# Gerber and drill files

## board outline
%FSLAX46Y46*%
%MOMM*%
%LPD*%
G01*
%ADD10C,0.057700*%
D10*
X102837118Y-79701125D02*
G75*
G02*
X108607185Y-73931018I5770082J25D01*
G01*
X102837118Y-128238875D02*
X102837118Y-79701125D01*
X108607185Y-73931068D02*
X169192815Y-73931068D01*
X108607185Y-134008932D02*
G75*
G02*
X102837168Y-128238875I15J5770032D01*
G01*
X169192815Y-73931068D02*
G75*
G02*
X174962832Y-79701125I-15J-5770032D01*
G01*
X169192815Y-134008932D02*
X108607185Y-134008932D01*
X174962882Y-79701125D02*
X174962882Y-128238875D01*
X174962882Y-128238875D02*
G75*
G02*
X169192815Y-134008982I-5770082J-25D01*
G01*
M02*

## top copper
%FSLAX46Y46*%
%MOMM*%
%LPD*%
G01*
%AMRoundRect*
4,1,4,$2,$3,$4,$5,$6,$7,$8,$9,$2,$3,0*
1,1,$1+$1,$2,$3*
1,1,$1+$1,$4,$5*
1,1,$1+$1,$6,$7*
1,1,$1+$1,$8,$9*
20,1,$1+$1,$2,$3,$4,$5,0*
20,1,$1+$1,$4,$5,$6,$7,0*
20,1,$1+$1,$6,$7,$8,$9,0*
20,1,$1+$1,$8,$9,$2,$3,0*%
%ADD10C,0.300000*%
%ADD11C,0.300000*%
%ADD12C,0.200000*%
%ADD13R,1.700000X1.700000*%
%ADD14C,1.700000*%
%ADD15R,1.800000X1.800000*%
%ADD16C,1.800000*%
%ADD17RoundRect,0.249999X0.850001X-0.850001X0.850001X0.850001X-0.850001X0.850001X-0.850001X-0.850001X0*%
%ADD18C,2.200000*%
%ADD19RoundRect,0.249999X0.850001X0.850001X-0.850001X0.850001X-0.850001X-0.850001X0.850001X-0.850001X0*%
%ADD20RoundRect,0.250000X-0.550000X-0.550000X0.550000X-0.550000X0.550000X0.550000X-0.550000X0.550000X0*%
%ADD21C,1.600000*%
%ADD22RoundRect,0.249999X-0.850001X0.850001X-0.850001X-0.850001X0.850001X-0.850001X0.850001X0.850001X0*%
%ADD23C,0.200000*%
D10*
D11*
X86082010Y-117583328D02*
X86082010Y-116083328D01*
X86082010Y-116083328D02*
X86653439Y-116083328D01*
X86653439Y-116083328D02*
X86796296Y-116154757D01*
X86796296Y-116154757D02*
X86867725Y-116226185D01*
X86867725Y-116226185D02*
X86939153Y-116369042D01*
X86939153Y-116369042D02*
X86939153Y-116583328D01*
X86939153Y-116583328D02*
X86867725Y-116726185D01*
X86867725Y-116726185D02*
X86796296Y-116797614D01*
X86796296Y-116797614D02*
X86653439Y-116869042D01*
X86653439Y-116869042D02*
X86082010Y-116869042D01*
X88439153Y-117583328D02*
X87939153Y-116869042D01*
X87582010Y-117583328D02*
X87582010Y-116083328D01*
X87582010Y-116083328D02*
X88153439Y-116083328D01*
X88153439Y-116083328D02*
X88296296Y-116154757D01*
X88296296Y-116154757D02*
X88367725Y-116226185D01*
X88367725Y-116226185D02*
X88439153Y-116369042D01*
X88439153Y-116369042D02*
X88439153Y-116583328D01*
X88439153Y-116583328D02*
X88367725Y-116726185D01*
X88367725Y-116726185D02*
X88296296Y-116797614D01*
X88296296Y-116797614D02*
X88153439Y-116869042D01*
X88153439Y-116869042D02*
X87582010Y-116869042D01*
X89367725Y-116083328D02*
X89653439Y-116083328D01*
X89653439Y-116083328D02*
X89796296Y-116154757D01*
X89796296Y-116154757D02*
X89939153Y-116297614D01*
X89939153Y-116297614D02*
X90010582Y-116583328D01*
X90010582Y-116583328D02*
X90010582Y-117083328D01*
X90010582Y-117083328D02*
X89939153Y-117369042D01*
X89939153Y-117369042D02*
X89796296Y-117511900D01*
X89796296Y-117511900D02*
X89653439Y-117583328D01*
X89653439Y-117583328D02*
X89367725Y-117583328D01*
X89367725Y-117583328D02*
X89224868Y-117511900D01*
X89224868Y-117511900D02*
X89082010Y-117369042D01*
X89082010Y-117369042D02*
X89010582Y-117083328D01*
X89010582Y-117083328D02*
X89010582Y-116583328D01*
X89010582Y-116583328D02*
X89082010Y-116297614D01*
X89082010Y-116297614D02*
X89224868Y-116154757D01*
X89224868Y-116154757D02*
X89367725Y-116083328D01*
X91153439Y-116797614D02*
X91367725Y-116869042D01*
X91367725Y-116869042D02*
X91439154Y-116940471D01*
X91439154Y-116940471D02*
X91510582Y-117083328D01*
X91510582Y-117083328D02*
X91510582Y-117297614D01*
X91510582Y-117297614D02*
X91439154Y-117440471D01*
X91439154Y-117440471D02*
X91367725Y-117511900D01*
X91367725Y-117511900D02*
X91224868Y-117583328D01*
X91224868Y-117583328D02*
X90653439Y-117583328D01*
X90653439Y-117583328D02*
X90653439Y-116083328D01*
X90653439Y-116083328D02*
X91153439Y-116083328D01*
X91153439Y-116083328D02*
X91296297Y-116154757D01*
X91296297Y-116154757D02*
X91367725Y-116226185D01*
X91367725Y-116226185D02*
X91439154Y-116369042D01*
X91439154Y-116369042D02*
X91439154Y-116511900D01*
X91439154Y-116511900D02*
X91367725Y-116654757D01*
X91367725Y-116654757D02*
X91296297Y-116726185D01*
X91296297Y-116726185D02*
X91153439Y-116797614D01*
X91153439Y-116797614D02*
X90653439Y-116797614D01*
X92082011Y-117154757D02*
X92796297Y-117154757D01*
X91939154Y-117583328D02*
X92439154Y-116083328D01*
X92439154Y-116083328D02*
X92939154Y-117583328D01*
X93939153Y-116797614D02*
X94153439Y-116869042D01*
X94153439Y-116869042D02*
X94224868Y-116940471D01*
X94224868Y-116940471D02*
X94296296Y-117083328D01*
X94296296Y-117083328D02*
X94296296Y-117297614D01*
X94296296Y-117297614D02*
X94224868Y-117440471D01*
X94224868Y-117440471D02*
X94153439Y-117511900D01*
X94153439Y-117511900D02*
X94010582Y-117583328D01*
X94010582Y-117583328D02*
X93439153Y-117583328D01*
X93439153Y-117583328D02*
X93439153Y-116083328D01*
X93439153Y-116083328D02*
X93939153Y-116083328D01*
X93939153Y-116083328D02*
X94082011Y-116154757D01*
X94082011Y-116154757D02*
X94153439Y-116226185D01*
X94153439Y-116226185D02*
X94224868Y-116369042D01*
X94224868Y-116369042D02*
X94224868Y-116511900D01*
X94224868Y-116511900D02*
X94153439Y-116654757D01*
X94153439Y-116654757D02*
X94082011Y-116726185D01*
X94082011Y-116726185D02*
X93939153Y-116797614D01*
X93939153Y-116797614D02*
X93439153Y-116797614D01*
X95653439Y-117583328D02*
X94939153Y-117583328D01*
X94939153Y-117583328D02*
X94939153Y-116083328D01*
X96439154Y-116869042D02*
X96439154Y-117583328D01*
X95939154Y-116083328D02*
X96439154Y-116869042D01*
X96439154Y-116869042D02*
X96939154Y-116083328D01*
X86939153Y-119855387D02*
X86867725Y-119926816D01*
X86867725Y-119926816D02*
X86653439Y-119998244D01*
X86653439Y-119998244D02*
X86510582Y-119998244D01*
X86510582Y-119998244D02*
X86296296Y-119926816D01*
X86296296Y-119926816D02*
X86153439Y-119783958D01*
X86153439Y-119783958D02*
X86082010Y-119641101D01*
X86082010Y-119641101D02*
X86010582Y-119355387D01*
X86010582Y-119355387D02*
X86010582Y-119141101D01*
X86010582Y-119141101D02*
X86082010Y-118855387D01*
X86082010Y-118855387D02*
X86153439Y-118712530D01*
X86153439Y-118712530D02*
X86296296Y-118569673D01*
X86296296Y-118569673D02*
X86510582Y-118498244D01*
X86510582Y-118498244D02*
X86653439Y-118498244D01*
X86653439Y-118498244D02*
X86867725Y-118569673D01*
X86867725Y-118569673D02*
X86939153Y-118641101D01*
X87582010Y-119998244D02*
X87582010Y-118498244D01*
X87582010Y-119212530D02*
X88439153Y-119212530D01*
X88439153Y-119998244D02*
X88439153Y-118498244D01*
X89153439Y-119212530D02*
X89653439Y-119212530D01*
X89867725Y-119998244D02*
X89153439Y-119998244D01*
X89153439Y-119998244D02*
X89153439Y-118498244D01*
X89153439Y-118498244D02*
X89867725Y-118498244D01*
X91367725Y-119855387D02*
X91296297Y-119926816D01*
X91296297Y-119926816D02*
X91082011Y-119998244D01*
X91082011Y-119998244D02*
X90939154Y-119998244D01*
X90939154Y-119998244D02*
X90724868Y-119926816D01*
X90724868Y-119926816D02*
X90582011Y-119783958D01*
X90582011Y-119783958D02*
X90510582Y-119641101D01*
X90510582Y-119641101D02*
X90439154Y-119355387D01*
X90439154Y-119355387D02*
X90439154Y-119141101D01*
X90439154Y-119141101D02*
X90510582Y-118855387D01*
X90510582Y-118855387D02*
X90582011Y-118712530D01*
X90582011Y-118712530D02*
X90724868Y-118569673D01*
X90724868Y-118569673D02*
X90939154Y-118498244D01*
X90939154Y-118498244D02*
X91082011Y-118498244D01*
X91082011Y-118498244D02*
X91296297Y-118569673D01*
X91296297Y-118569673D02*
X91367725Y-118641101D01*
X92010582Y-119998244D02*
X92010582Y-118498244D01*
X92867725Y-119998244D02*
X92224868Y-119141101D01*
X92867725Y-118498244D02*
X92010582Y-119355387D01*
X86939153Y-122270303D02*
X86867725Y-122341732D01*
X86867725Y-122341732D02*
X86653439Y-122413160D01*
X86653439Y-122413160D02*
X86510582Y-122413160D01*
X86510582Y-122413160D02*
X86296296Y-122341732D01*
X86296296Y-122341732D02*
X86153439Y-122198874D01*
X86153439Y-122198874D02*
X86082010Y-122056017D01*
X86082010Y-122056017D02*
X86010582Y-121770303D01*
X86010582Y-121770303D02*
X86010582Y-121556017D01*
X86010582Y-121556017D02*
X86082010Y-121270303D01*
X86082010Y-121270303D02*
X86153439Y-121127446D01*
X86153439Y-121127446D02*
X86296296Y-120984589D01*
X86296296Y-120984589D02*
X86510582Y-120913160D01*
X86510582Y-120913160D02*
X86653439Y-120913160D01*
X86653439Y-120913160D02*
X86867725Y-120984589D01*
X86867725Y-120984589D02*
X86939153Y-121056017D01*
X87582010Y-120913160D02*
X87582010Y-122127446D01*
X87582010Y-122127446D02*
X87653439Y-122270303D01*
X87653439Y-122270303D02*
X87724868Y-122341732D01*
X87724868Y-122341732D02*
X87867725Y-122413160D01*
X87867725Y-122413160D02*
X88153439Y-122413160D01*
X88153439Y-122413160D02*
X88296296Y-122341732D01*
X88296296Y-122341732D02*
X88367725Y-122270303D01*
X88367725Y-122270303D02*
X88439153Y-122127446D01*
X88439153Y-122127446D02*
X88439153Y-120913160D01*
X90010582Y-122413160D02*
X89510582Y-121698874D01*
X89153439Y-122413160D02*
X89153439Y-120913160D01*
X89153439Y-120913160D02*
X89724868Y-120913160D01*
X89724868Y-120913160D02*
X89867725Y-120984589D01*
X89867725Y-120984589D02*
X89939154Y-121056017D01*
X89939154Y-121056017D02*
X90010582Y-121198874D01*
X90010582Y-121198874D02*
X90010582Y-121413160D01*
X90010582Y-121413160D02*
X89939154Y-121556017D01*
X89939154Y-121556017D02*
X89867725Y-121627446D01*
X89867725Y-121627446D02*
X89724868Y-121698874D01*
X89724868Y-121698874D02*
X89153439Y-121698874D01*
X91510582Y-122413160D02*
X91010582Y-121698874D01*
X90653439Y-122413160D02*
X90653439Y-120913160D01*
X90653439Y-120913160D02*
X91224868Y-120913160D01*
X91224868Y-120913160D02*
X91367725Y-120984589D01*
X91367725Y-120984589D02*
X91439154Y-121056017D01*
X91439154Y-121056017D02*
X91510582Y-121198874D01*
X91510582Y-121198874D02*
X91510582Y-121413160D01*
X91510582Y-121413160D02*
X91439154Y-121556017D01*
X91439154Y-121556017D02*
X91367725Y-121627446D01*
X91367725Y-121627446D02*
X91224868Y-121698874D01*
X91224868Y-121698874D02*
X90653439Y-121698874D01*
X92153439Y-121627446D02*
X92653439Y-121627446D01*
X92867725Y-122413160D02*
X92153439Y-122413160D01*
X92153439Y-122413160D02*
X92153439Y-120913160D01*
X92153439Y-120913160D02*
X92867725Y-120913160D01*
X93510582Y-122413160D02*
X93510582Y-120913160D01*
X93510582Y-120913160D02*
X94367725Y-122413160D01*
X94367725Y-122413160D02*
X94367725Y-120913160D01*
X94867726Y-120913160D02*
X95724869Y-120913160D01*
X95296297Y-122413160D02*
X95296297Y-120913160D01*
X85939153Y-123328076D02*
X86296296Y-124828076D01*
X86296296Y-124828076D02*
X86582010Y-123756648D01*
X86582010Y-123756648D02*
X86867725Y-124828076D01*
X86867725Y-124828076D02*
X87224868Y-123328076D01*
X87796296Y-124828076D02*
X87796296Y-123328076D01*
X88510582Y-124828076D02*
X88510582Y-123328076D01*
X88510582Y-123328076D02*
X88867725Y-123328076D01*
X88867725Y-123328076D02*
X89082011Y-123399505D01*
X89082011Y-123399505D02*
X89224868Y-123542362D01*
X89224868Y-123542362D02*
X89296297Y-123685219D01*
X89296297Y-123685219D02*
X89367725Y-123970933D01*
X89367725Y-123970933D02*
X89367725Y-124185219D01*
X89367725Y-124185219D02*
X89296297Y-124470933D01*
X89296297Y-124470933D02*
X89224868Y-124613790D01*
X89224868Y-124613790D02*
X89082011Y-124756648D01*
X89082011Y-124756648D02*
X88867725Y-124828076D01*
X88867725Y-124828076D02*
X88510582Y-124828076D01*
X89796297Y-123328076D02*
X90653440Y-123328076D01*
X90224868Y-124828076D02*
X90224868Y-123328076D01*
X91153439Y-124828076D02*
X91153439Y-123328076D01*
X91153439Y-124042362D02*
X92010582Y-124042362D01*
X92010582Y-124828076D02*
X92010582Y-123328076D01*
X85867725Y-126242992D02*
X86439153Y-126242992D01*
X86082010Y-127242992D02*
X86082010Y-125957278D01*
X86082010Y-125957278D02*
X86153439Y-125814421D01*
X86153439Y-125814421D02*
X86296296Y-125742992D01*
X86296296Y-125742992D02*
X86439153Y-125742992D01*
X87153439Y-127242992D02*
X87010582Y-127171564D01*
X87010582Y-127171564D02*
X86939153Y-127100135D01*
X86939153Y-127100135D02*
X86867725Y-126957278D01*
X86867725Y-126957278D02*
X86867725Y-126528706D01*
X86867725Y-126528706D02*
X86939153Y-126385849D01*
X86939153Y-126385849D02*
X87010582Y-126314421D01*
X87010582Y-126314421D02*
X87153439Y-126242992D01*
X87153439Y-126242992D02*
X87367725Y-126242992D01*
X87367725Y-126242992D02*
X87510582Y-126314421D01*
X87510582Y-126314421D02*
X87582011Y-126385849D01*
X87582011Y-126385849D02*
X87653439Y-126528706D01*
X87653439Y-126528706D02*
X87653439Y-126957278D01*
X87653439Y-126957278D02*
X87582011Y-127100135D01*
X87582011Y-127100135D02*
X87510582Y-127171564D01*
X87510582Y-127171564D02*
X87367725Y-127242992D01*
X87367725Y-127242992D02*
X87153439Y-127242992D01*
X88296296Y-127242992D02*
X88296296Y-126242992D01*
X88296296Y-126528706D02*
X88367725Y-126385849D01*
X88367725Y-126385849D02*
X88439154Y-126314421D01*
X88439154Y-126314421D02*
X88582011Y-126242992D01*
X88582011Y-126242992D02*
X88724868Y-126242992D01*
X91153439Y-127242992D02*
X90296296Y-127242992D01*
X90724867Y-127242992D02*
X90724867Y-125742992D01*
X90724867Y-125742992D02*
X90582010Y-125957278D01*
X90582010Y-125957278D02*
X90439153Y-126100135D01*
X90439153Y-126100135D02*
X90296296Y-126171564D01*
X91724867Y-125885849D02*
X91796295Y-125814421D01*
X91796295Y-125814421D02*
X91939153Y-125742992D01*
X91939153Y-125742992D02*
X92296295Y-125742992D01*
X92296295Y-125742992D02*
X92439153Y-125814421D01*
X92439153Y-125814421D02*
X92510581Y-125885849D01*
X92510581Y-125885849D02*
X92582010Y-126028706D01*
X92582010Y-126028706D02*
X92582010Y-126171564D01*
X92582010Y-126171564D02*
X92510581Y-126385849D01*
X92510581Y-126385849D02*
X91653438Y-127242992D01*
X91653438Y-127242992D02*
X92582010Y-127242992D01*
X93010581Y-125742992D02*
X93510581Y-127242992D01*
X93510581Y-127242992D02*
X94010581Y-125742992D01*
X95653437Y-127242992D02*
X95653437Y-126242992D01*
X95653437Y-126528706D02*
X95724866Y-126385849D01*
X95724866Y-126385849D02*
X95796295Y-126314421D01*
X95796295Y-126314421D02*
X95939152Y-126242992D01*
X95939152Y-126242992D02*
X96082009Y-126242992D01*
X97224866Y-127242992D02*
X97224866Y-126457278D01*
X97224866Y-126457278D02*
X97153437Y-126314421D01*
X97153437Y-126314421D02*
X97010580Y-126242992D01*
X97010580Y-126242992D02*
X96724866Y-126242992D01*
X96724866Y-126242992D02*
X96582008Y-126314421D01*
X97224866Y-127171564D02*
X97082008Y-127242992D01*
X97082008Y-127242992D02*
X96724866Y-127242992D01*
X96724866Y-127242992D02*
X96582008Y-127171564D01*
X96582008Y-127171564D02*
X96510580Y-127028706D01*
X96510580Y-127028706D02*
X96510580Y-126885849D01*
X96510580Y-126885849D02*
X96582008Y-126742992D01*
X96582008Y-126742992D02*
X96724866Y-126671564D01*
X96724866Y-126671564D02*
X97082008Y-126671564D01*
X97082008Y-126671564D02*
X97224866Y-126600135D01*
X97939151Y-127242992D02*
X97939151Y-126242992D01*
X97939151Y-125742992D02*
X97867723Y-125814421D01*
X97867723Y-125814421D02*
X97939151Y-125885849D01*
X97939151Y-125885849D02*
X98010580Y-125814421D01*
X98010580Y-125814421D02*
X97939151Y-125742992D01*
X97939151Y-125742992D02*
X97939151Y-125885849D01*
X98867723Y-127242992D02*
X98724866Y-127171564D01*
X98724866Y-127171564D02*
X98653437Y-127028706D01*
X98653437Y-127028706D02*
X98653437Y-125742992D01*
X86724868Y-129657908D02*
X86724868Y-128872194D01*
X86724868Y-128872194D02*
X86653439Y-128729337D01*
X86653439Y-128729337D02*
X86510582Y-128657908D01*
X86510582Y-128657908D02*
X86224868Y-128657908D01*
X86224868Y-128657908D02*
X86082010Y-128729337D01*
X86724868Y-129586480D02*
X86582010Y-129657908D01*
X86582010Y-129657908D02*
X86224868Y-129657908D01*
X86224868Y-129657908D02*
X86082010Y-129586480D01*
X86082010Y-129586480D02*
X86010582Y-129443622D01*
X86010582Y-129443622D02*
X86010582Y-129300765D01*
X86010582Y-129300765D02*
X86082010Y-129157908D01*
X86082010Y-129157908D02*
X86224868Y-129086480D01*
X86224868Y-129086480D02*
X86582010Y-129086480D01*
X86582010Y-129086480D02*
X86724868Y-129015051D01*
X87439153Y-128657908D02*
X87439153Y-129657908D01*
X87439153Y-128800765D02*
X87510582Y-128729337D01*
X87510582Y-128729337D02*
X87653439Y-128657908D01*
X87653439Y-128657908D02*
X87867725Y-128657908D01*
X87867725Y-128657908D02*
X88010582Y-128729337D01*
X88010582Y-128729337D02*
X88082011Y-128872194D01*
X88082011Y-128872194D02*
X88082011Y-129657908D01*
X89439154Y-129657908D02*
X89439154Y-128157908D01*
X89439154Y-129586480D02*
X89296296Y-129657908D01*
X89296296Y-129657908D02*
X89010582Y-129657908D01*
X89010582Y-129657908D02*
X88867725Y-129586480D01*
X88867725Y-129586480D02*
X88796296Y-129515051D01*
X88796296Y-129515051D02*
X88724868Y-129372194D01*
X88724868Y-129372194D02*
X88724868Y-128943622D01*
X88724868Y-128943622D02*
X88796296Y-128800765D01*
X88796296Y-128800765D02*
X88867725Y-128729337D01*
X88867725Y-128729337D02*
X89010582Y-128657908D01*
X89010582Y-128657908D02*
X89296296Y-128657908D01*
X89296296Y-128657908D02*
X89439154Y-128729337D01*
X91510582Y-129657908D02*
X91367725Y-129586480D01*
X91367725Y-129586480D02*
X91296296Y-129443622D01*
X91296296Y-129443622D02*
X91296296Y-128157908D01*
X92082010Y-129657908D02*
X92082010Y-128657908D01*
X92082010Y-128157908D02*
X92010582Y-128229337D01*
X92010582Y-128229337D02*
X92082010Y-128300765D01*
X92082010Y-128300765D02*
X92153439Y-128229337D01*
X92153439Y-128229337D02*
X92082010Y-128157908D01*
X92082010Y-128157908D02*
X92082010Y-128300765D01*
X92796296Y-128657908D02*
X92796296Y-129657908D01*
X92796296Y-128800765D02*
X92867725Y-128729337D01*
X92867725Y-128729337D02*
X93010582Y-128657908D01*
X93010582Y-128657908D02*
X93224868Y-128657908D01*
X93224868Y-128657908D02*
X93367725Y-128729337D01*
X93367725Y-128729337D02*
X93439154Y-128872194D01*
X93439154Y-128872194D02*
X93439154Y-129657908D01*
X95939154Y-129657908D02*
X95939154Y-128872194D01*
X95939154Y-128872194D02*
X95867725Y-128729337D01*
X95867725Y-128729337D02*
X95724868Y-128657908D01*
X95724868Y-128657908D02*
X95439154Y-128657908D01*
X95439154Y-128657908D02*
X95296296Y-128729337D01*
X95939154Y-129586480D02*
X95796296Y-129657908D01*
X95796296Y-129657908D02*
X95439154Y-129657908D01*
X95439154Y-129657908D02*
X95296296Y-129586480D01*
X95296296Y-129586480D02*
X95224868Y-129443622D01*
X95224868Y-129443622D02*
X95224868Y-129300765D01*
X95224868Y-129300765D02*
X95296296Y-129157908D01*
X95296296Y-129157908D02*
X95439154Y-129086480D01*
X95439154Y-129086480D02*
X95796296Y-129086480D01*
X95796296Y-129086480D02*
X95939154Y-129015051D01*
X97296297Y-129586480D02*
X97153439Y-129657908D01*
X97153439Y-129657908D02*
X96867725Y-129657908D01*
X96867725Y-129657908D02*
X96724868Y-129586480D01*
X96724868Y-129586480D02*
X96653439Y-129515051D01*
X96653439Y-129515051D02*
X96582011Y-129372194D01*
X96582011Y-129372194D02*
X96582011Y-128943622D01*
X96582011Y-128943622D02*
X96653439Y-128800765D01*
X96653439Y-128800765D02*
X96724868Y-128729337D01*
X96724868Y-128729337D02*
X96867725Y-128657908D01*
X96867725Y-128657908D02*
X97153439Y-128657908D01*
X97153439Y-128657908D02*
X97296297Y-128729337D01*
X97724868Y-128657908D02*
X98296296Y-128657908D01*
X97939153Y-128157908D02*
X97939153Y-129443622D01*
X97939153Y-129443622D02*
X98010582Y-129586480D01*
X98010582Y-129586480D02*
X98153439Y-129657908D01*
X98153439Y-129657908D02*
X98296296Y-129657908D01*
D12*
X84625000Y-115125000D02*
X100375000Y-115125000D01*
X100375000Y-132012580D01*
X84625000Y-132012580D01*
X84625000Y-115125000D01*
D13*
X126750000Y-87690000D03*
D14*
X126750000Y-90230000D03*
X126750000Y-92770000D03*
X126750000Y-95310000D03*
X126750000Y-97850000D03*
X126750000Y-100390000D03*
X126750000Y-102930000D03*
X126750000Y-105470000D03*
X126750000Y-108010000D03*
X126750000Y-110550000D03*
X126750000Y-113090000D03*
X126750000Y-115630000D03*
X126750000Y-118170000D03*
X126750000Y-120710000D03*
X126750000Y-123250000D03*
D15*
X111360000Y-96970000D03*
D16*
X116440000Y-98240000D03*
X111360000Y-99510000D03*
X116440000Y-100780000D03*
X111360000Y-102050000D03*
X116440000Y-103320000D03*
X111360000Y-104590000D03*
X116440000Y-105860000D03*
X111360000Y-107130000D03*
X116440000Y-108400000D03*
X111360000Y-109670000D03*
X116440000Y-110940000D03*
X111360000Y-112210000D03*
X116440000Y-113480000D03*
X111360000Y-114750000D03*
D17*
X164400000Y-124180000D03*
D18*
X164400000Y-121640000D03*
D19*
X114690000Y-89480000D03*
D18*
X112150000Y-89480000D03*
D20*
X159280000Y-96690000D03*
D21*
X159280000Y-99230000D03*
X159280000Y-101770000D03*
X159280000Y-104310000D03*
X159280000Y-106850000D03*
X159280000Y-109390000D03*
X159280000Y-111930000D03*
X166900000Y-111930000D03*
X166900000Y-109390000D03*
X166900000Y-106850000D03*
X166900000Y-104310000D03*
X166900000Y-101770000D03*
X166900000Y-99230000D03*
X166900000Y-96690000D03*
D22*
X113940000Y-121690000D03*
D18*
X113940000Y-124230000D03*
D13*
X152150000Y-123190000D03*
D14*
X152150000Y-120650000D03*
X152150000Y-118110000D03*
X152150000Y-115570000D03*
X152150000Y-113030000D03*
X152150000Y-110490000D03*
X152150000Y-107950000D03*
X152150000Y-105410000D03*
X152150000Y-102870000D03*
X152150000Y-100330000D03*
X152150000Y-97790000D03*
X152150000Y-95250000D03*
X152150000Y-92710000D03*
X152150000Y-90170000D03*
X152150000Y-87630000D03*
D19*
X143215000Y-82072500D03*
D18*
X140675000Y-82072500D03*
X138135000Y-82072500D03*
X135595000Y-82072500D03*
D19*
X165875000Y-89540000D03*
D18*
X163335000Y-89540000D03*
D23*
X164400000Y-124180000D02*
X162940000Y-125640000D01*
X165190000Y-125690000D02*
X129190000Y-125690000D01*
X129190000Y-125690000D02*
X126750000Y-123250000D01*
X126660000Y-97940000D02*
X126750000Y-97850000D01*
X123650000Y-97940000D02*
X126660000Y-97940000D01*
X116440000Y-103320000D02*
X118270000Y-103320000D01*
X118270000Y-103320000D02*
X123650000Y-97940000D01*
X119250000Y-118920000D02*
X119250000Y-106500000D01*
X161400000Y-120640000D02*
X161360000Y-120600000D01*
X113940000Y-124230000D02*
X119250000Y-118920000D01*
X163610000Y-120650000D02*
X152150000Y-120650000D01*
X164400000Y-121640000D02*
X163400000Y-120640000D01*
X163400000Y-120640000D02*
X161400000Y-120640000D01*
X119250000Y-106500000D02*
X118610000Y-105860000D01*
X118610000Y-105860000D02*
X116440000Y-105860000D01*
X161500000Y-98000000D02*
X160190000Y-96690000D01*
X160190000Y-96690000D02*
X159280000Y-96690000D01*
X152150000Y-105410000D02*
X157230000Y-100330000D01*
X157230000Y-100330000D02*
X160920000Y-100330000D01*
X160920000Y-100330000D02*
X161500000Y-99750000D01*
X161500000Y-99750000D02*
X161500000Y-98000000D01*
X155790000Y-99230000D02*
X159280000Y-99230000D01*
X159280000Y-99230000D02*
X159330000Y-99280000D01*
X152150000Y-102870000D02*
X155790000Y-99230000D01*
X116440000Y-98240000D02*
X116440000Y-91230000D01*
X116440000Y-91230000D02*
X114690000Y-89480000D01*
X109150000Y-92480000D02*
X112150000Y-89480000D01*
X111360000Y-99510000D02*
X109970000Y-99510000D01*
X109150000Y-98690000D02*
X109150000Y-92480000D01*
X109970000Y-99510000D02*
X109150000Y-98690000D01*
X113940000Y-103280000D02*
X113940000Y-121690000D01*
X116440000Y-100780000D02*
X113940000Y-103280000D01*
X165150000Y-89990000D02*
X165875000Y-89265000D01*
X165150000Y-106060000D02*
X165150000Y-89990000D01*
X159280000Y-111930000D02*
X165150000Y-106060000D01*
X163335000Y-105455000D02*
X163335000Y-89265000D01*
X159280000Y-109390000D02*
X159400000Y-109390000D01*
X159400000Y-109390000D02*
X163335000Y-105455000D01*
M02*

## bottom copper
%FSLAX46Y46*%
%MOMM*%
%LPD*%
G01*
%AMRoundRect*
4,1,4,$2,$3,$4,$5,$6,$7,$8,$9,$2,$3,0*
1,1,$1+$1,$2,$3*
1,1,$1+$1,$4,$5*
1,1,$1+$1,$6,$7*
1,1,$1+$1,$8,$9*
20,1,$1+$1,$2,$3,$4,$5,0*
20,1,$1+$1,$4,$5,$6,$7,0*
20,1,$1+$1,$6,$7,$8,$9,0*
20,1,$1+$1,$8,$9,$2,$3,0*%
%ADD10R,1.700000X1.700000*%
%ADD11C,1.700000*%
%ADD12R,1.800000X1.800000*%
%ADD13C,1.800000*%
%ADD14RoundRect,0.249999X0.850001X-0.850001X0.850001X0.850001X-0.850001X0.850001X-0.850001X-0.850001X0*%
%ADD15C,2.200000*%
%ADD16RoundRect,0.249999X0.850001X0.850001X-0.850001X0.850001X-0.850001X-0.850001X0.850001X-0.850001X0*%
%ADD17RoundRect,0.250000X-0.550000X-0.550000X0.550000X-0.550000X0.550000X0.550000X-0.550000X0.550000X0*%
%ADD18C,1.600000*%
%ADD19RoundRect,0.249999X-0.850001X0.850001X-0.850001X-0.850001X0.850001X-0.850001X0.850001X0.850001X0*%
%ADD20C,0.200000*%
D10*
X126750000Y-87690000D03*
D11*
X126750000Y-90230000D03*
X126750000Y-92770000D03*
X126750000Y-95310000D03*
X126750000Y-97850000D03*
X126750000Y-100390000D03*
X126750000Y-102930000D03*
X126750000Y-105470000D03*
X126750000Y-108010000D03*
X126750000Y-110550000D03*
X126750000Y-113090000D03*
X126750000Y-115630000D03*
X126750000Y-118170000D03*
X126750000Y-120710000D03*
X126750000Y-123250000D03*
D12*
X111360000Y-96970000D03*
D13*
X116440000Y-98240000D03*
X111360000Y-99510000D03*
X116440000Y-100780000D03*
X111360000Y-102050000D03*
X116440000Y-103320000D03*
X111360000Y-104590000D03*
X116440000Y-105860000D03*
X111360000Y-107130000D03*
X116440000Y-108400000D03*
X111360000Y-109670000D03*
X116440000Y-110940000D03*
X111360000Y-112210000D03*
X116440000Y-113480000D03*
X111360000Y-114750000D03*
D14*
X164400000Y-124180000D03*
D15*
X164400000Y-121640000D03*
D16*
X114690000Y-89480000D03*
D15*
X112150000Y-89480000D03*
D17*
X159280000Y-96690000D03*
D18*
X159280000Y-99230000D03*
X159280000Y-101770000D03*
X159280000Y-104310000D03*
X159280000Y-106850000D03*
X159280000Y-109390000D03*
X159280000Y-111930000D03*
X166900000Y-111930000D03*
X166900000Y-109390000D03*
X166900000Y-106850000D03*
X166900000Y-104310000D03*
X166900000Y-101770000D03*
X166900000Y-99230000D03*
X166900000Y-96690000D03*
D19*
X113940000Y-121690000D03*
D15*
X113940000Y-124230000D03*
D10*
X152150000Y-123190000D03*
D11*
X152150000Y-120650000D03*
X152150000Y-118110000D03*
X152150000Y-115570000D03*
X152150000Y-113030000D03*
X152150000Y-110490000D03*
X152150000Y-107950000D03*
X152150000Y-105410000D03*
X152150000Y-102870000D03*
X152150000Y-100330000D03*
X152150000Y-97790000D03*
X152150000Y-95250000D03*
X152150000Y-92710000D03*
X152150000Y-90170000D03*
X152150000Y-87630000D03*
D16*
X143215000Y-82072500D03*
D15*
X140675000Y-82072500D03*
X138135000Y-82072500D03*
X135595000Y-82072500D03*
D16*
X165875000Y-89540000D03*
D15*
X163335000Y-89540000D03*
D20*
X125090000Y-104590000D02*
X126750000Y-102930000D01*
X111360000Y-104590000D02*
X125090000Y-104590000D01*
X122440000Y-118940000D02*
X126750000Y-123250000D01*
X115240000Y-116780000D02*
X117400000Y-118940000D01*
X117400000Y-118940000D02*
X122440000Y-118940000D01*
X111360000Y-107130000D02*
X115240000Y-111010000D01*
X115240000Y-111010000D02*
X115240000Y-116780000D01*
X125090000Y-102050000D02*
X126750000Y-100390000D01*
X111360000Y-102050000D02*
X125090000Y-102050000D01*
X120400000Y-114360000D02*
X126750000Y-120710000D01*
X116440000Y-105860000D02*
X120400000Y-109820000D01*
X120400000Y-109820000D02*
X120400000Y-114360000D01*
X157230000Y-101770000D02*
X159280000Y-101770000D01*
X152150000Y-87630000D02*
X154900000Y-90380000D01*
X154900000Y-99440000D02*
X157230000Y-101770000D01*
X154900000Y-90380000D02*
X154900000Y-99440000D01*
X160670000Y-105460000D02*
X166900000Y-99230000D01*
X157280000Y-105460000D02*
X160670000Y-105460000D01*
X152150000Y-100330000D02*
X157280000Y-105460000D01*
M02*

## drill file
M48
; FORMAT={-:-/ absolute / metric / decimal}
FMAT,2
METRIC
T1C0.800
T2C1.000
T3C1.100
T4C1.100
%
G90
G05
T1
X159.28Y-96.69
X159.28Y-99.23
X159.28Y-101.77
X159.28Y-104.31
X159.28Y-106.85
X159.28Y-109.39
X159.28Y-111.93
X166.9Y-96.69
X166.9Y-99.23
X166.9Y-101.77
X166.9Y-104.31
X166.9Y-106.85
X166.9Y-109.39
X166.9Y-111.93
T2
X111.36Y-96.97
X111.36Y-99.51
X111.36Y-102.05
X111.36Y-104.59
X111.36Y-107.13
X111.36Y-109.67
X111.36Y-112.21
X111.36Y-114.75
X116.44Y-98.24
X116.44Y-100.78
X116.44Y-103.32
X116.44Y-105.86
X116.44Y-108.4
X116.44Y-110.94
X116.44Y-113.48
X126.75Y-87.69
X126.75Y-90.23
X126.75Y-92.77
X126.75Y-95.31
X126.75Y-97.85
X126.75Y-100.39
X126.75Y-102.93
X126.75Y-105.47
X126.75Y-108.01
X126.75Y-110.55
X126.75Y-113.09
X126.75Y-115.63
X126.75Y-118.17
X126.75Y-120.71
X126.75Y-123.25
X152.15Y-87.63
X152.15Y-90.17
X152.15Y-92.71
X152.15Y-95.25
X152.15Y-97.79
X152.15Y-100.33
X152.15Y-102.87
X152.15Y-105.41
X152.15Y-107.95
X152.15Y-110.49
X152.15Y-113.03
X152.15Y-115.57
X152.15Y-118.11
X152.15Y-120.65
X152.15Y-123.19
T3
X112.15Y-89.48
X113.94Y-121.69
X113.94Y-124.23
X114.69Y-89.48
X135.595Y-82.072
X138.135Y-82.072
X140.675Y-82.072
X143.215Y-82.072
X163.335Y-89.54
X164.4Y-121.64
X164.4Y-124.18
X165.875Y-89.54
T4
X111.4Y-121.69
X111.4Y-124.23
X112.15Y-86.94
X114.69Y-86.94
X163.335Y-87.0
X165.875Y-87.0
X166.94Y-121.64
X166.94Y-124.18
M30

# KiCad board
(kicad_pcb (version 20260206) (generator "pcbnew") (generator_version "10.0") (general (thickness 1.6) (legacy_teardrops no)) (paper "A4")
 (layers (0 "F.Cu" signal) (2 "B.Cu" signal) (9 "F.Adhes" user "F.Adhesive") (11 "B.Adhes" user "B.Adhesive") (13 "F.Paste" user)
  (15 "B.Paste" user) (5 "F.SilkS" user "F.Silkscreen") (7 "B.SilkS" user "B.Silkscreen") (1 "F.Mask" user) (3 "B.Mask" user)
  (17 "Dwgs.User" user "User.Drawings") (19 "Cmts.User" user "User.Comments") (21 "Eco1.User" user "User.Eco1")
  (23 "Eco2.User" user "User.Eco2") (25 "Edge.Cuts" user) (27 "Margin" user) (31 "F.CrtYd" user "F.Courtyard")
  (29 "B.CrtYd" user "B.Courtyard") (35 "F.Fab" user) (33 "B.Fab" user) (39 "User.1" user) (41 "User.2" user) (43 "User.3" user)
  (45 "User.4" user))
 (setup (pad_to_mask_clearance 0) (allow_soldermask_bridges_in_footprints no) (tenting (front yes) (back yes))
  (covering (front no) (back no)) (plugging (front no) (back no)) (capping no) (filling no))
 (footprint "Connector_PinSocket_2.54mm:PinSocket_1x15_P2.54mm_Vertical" (layer "F.Cu") (at 126.75 87.69)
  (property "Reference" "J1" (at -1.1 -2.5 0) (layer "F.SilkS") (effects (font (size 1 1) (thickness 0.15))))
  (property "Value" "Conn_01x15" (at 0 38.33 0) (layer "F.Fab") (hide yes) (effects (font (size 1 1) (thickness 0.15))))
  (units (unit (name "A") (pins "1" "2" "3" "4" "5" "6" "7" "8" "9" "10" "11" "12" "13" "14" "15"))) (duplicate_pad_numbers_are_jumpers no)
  (pad "1" thru_hole rect (at 0 0) (size 1.7 1.7) (drill 1) (layers "*.Cu" "*.Mask") (remove_unused_layers no) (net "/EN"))
  (pad "2" thru_hole circle (at 0 2.54) (size 1.7 1.7) (drill 1) (layers "*.Cu" "*.Mask") (remove_unused_layers no) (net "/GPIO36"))
  (pad "3" thru_hole circle (at 0 5.08) (size 1.7 1.7) (drill 1) (layers "*.Cu" "*.Mask") (remove_unused_layers no) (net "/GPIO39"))
  (pad "4" thru_hole circle (at 0 7.62) (size 1.7 1.7) (drill 1) (layers "*.Cu" "*.Mask") (remove_unused_layers no) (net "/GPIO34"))
  (pad "5" thru_hole circle (at 0 10.16) (size 1.7 1.7) (drill 1) (layers "*.Cu" "*.Mask") (remove_unused_layers no) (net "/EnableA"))
  (pad "6" thru_hole circle (at 0 12.7) (size 1.7 1.7) (drill 1) (layers "*.Cu" "*.Mask") (remove_unused_layers no) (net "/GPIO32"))
  (pad "7" thru_hole circle (at 0 15.24) (size 1.7 1.7) (drill 1) (layers "*.Cu" "*.Mask") (remove_unused_layers no) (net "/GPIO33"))
  (pad "8" thru_hole circle (at 0 17.78) (size 1.7 1.7) (drill 1) (layers "*.Cu" "*.Mask") (remove_unused_layers no) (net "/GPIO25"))
  (pad "9" thru_hole circle (at 0 20.32) (size 1.7 1.7) (drill 1) (layers "*.Cu" "*.Mask") (remove_unused_layers no) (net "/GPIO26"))
  (pad "10" thru_hole circle (at 0 22.86) (size 1.7 1.7) (drill 1) (layers "*.Cu" "*.Mask") (remove_unused_layers no) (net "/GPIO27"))
  (pad "11" thru_hole circle (at 0 25.4) (size 1.7 1.7) (drill 1) (layers "*.Cu" "*.Mask") (remove_unused_layers no) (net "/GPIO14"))
  (pad "12" thru_hole circle (at 0 27.94) (size 1.7 1.7) (drill 1) (layers "*.Cu" "*.Mask") (remove_unused_layers no) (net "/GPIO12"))
  (pad "13" thru_hole circle (at 0 30.48) (size 1.7 1.7) (drill 1) (layers "*.Cu" "*.Mask") (remove_unused_layers no) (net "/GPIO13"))
  (pad "14" thru_hole circle (at 0 33.02) (size 1.7 1.7) (drill 1) (layers "*.Cu" "*.Mask") (remove_unused_layers no) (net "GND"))
  (pad "15" thru_hole circle (at 0 35.56) (size 1.7 1.7) (drill 1) (layers "*.Cu" "*.Mask") (remove_unused_layers no) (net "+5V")))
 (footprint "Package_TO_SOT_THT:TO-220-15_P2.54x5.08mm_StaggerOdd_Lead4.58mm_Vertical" (layer "F.Cu") (at 111.36 96.97 -90)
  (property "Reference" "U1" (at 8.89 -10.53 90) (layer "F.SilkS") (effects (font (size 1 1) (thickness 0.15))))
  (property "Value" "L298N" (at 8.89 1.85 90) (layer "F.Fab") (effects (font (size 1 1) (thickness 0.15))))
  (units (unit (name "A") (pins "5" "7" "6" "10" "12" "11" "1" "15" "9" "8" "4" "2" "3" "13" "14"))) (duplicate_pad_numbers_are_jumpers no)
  (pad "1" thru_hole rect (at 0 0 270) (size 1.8 1.8) (drill 1) (layers "*.Cu" "*.Mask") (remove_unused_layers no)
   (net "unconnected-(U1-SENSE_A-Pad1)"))
  (pad "2" thru_hole circle (at 1.27 -5.08 270) (size 1.8 1.8) (drill 1) (layers "*.Cu" "*.Mask") (remove_unused_layers no)
   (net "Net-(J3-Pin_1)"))
  (pad "3" thru_hole circle (at 2.54 0 270) (size 1.8 1.8) (drill 1) (layers "*.Cu" "*.Mask") (remove_unused_layers no)
   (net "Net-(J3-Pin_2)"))
  (pad "4" thru_hole circle (at 3.81 -5.08 270) (size 1.8 1.8) (drill 1) (layers "*.Cu" "*.Mask") (remove_unused_layers no) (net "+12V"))
  (pad "5" thru_hole circle (at 5.08 0 270) (size 1.8 1.8) (drill 1) (layers "*.Cu" "*.Mask") (remove_unused_layers no) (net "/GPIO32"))
  (pad "6" thru_hole circle (at 6.35 -5.08 270) (size 1.8 1.8) (drill 1) (layers "*.Cu" "*.Mask") (remove_unused_layers no) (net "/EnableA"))
  (pad "7" thru_hole circle (at 7.62 0 270) (size 1.8 1.8) (drill 1) (layers "*.Cu" "*.Mask") (remove_unused_layers no) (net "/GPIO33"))
  (pad "8" thru_hole circle (at 8.89 -5.08 270) (size 1.8 1.8) (drill 1) (layers "*.Cu" "*.Mask") (remove_unused_layers no) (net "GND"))
  (pad "9" thru_hole circle (at 10.16 0 270) (size 1.8 1.8) (drill 1) (layers "*.Cu" "*.Mask") (remove_unused_layers no) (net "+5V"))
  (pad "10" thru_hole circle (at 11.43 -5.08 270) (size 1.8 1.8) (drill 1) (layers "*.Cu" "*.Mask") (remove_unused_layers no)
   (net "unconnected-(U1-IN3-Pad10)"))
  (pad "11" thru_hole circle (at 12.7 0 270) (size 1.8 1.8) (drill 1) (layers "*.Cu" "*.Mask") (remove_unused_layers no)
   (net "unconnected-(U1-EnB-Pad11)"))
  (pad "12" thru_hole circle (at 13.97 -5.08 270) (size 1.8 1.8) (drill 1) (layers "*.Cu" "*.Mask") (remove_unused_layers no)
   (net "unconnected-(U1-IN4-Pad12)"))
  (pad "13" thru_hole circle (at 15.24 0 270) (size 1.8 1.8) (drill 1) (layers "*.Cu" "*.Mask") (remove_unused_layers no)
   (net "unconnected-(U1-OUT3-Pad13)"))
  (pad "14" thru_hole circle (at 16.51 -5.08 270) (size 1.8 1.8) (drill 1) (layers "*.Cu" "*.Mask") (remove_unused_layers no)
   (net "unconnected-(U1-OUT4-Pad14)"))
  (pad "15" thru_hole circle (at 17.78 0 270) (size 1.8 1.8) (drill 1) (layers "*.Cu" "*.Mask") (remove_unused_layers no)
   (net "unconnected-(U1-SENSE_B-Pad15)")))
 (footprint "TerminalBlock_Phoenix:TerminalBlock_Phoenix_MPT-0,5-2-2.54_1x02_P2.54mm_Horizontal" (layer "F.Cu") (at 164.4 124.18 90)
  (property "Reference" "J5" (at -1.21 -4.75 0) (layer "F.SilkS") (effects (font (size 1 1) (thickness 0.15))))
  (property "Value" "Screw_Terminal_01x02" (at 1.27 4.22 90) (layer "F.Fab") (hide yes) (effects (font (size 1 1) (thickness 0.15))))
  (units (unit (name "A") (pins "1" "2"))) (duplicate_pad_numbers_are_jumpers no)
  (pad "" np_thru_hole circle (at 0 2.54 90) (size 1.1 1.1) (drill 1.1) (layers "*.Cu" "*.Mask"))
  (pad "" np_thru_hole circle (at 2.54 2.54 90) (size 1.1 1.1) (drill 1.1) (layers "*.Cu" "*.Mask"))
  (pad "1" thru_hole roundrect (at 0 0 90) (size 2.2 2.2) (drill 1.1) (layers "*.Cu" "*.Mask") (remove_unused_layers no)
   (roundrect_rratio 0.113636) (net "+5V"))
  (pad "2" thru_hole circle (at 2.54 0 90) (size 2.2 2.2) (drill 1.1) (layers "*.Cu" "*.Mask") (remove_unused_layers no) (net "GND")))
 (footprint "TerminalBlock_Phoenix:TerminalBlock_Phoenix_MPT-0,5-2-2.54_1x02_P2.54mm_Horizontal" (layer "F.Cu") (at 114.69 89.48 180)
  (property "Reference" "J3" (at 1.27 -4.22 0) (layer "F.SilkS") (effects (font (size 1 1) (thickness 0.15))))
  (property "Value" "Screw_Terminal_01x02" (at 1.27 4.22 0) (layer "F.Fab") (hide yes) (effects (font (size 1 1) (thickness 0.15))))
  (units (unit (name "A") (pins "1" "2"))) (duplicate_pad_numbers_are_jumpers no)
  (pad "" np_thru_hole circle (at 0 2.54 180) (size 1.1 1.1) (drill 1.1) (layers "*.Cu" "*.Mask"))
  (pad "" np_thru_hole circle (at 2.54 2.54 180) (size 1.1 1.1) (drill 1.1) (layers "*.Cu" "*.Mask"))
  (pad "1" thru_hole roundrect (at 0 0 180) (size 2.2 2.2) (drill 1.1) (layers "*.Cu" "*.Mask") (remove_unused_layers no)
   (roundrect_rratio 0.113636) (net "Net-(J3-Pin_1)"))
  (pad "2" thru_hole circle (at 2.54 0 180) (size 2.2 2.2) (drill 1.1) (layers "*.Cu" "*.Mask") (remove_unused_layers no)
   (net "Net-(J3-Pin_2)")))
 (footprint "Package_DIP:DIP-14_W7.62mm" (layer "F.Cu") (at 159.28 96.69)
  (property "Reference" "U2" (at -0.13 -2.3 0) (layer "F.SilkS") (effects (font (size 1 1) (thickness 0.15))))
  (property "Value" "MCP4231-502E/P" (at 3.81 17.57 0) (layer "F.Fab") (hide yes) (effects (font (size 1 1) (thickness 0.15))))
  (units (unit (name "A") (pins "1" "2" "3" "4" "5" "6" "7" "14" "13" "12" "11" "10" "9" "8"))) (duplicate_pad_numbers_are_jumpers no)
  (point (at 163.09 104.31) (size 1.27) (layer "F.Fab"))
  (pad "1" thru_hole roundrect (at 0 0) (size 1.6 1.6) (drill 0.8) (layers "*.Cu" "*.Mask") (remove_unused_layers no)
   (roundrect_rratio 0.15625) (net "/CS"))
  (pad "2" thru_hole circle (at 0 2.54) (size 1.6 1.6) (drill 0.8) (layers "*.Cu" "*.Mask") (remove_unused_layers no) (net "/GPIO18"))
  (pad "3" thru_hole circle (at 0 5.08) (size 1.6 1.6) (drill 0.8) (layers "*.Cu" "*.Mask") (remove_unused_layers no) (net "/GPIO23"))
  (pad "4" thru_hole circle (at 0 7.62) (size 1.6 1.6) (drill 0.8) (layers "*.Cu" "*.Mask") (remove_unused_layers no) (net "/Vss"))
  (pad "5" thru_hole circle (at 0 10.16) (size 1.6 1.6) (drill 0.8) (layers "*.Cu" "*.Mask") (remove_unused_layers no)
   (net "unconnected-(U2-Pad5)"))
  (pad "6" thru_hole circle (at 0 12.7) (size 1.6 1.6) (drill 0.8) (layers "*.Cu" "*.Mask") (remove_unused_layers no) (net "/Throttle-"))
  (pad "7" thru_hole circle (at 0 15.24) (size 1.6 1.6) (drill 0.8) (layers "*.Cu" "*.Mask") (remove_unused_layers no) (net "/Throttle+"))
  (pad "8" thru_hole circle (at 7.62 15.24) (size 1.6 1.6) (drill 0.8) (layers "*.Cu" "*.Mask") (remove_unused_layers no)
   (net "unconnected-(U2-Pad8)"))
  (pad "9" thru_hole circle (at 7.62 12.7) (size 1.6 1.6) (drill 0.8) (layers "*.Cu" "*.Mask") (remove_unused_layers no)
   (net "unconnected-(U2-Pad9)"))
  (pad "10" thru_hole circle (at 7.62 10.16) (size 1.6 1.6) (drill 0.8) (layers "*.Cu" "*.Mask") (remove_unused_layers no)
   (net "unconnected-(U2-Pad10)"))
  (pad "11" thru_hole circle (at 7.62 7.62) (size 1.6 1.6) (drill 0.8) (layers "*.Cu" "*.Mask") (remove_unused_layers no) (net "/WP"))
  (pad "12" thru_hole circle (at 7.62 5.08) (size 1.6 1.6) (drill 0.8) (layers "*.Cu" "*.Mask") (remove_unused_layers no) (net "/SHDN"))
  (pad "13" thru_hole circle (at 7.62 2.54) (size 1.6 1.6) (drill 0.8) (layers "*.Cu" "*.Mask") (remove_unused_layers no) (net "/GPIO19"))
  (pad "14" thru_hole circle (at 7.62 0) (size 1.6 1.6) (drill 0.8) (layers "*.Cu" "*.Mask") (remove_unused_layers no) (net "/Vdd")))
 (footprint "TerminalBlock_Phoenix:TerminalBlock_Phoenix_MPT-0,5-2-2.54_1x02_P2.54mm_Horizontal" (layer "F.Cu") (at 113.94 121.69 -90)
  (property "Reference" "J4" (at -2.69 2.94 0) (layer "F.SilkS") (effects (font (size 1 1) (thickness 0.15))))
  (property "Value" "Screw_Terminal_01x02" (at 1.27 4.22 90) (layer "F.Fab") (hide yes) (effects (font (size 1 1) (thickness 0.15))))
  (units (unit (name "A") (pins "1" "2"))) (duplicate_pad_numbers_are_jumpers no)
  (pad "" np_thru_hole circle (at 0 2.54 270) (size 1.1 1.1) (drill 1.1) (layers "*.Cu" "*.Mask"))
  (pad "" np_thru_hole circle (at 2.54 2.54 270) (size 1.1 1.1) (drill 1.1) (layers "*.Cu" "*.Mask"))
  (pad "1" thru_hole roundrect (at 0 0 270) (size 2.2 2.2) (drill 1.1) (layers "*.Cu" "*.Mask") (remove_unused_layers no)
   (roundrect_rratio 0.113636) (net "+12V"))
  (pad "2" thru_hole circle (at 2.54 0 270) (size 2.2 2.2) (drill 1.1) (layers "*.Cu" "*.Mask") (remove_unused_layers no) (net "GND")))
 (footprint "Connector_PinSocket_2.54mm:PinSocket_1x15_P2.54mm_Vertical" (layer "F.Cu") (at 152.15 123.19 180)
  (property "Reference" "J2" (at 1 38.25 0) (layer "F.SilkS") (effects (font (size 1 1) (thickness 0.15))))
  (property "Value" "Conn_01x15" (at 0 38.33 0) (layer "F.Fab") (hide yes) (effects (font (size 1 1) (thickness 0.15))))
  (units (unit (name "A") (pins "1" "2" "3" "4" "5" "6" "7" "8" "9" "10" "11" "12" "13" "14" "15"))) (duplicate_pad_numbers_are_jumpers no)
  (pad "1" thru_hole rect (at 0 0 180) (size 1.7 1.7) (drill 1) (layers "*.Cu" "*.Mask") (remove_unused_layers no) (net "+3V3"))
  (pad "2" thru_hole circle (at 0 2.54 180) (size 1.7 1.7) (drill 1) (layers "*.Cu" "*.Mask") (remove_unused_layers no) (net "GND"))
  (pad "3" thru_hole circle (at 0 5.08 180) (size 1.7 1.7) (drill 1) (layers "*.Cu" "*.Mask") (remove_unused_layers no) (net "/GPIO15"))
  (pad "4" thru_hole circle (at 0 7.62 180) (size 1.7 1.7) (drill 1) (layers "*.Cu" "*.Mask") (remove_unused_layers no) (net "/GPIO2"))
  (pad "5" thru_hole circle (at 0 10.16 180) (size 1.7 1.7) (drill 1) (layers "*.Cu" "*.Mask") (remove_unused_layers no) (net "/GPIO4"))
  (pad "6" thru_hole circle (at 0 12.7 180) (size 1.7 1.7) (drill 1) (layers "*.Cu" "*.Mask") (remove_unused_layers no) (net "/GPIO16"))
  (pad "7" thru_hole circle (at 0 15.24 180) (size 1.7 1.7) (drill 1) (layers "*.Cu" "*.Mask") (remove_unused_layers no) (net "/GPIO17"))
  (pad "8" thru_hole circle (at 0 17.78 180) (size 1.7 1.7) (drill 1) (layers "*.Cu" "*.Mask") (remove_unused_layers no) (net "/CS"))
  (pad "9" thru_hole circle (at 0 20.32 180) (size 1.7 1.7) (drill 1) (layers "*.Cu" "*.Mask") (remove_unused_layers no) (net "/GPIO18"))
  (pad "10" thru_hole circle (at 0 22.86 180) (size 1.7 1.7) (drill 1) (layers "*.Cu" "*.Mask") (remove_unused_layers no) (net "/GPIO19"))
  (pad "11" thru_hole circle (at 0 25.4 180) (size 1.7 1.7) (drill 1) (layers "*.Cu" "*.Mask") (remove_unused_layers no) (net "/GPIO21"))
  (pad "12" thru_hole circle (at 0 27.94 180) (size 1.7 1.7) (drill 1) (layers "*.Cu" "*.Mask") (remove_unused_layers no) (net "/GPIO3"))
  (pad "13" thru_hole circle (at 0 30.48 180) (size 1.7 1.7) (drill 1) (layers "*.Cu" "*.Mask") (remove_unused_layers no) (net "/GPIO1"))
  (pad "14" thru_hole circle (at 0 33.02 180) (size 1.7 1.7) (drill 1) (layers "*.Cu" "*.Mask") (remove_unused_layers no) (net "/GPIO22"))
  (pad "15" thru_hole circle (at 0 35.56 180) (size 1.7 1.7) (drill 1) (layers "*.Cu" "*.Mask") (remove_unused_layers no) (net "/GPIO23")))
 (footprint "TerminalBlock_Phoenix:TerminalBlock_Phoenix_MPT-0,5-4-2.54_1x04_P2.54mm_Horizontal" (layer "F.Cu") (at 143.215 82.0725 180)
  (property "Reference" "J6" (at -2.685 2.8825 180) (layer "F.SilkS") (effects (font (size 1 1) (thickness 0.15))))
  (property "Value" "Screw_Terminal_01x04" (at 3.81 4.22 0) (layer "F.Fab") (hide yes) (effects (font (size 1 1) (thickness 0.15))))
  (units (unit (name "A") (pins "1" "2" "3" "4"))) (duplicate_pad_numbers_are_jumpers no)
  (pad "1" thru_hole roundrect (at 0 0 180) (size 2.2 2.2) (drill 1.1) (layers "*.Cu" "*.Mask") (remove_unused_layers no)
   (roundrect_rratio 0.113636) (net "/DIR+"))
  (pad "2" thru_hole circle (at 2.54 0 180) (size 2.2 2.2) (drill 1.1) (layers "*.Cu" "*.Mask") (remove_unused_layers no) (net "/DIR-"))
  (pad "3" thru_hole circle (at 5.08 0 180) (size 2.2 2.2) (drill 1.1) (layers "*.Cu" "*.Mask") (remove_unused_layers no) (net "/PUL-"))
  (pad "4" thru_hole circle (at 7.62 0 180) (size 2.2 2.2) (drill 1.1) (layers "*.Cu" "*.Mask") (remove_unused_layers no) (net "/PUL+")))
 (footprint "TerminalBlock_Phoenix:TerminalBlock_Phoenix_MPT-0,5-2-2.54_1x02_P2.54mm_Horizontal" (layer "F.Cu") (at 165.875 89.54 180)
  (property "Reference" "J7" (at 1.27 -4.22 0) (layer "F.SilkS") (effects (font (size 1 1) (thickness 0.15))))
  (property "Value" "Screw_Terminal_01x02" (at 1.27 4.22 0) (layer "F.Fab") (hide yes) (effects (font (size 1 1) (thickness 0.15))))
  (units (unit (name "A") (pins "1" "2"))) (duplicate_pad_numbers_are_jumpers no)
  (pad "" np_thru_hole circle (at 0 2.54 180) (size 1.1 1.1) (drill 1.1) (layers "*.Cu" "*.Mask"))
  (pad "" np_thru_hole circle (at 2.54 2.54 180) (size 1.1 1.1) (drill 1.1) (layers "*.Cu" "*.Mask"))
  (pad "1" thru_hole roundrect (at 0 0 180) (size 2.2 2.2) (drill 1.1) (layers "*.Cu" "*.Mask") (remove_unused_layers no)
   (roundrect_rratio 0.113636) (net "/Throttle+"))
  (pad "2" thru_hole circle (at 2.54 0 180) (size 2.2 2.2) (drill 1.1) (layers "*.Cu" "*.Mask") (remove_unused_layers no) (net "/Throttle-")))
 (gr_arc (start 102.837118 79.701125) (mid 104.527131 75.621071) (end 108.607185 73.931068) (stroke (width 0.0577) (type default))
  (layer "Edge.Cuts"))
 (gr_line (start 102.837118 128.238875) (end 102.837118 79.701125) (stroke (width 0.0577) (type default)) (layer "Edge.Cuts"))
 (gr_line (start 108.607185 73.931068) (end 169.192815 73.931068) (stroke (width 0.0577) (type default)) (layer "Edge.Cuts"))
 (gr_arc (start 108.607185 134.008932) (mid 104.527139 132.318921) (end 102.837118 128.238875) (stroke (width 0.0577) (type default))
  (layer "Edge.Cuts"))
 (gr_arc (start 169.192815 73.931068) (mid 173.272861 75.621079) (end 174.962882 79.701125) (stroke (width 0.0577) (type default))
  (layer "Edge.Cuts"))
 (gr_line (start 169.192815 134.008932) (end 108.607185 134.008932) (stroke (width 0.0577) (type default)) (layer "Edge.Cuts"))
 (gr_line (start 174.962882 79.701125) (end 174.962882 128.238875) (stroke (width 0.0577) (type default)) (layer "Edge.Cuts"))
 (gr_arc (start 174.962882 128.238875) (mid 173.272869 132.318929) (end 169.192815 134.008932) (stroke (width 0.0577) (type default))
  (layer "Edge.Cuts"))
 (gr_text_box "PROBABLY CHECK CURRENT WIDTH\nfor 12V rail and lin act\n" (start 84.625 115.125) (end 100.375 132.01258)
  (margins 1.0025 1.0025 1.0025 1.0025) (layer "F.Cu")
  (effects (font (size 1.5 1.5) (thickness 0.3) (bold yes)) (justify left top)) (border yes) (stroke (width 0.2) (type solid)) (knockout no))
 (segment (start 125.09 104.59) (end 126.75 102.93) (width 0.2) (layer "B.Cu") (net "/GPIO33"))
 (segment (start 111.36 104.59) (end 125.09 104.59) (width 0.2) (layer "B.Cu") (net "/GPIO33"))
 (segment (start 164.4 124.18) (end 162.94 125.64) (width 0.2) (layer "F.Cu") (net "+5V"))
 (segment (start 165.19 125.69) (end 129.19 125.69) (width 0.2) (layer "F.Cu") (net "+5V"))
 (segment (start 129.19 125.69) (end 126.75 123.25) (width 0.2) (layer "F.Cu") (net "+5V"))
 (segment (start 122.44 118.94) (end 126.75 123.25) (width 0.2) (layer "B.Cu") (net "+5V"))
 (segment (start 115.24 116.78) (end 117.4 118.94) (width 0.2) (layer "B.Cu") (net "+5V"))
 (segment (start 117.4 118.94) (end 122.44 118.94) (width 0.2) (layer "B.Cu") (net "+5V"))
 (segment (start 111.36 107.13) (end 115.24 111.01) (width 0.2) (layer "B.Cu") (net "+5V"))
 (segment (start 115.24 111.01) (end 115.24 116.78) (width 0.2) (layer "B.Cu") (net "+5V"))
 (segment (start 126.66 97.94) (end 126.75 97.85) (width 0.2) (layer "F.Cu") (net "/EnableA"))
 (segment (start 123.65 97.94) (end 126.66 97.94) (width 0.2) (layer "F.Cu") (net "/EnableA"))
 (segment (start 116.44 103.32) (end 118.27 103.32) (width 0.2) (layer "F.Cu") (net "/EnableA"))
 (segment (start 118.27 103.32) (end 123.65 97.94) (width 0.2) (layer "F.Cu") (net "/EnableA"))
 (segment (start 125.09 102.05) (end 126.75 100.39) (width 0.2) (layer "B.Cu") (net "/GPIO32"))
 (segment (start 111.36 102.05) (end 125.09 102.05) (width 0.2) (layer "B.Cu") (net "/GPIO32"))
 (segment (start 119.25 118.92) (end 119.25 106.5) (width 0.2) (layer "F.Cu") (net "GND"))
 (segment (start 161.4 120.64) (end 161.36 120.6) (width 0.2) (layer "F.Cu") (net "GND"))
 (segment (start 113.94 124.23) (end 119.25 118.92) (width 0.2) (layer "F.Cu") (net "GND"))
 (segment (start 163.61 120.65) (end 152.15 120.65) (width 0.2) (layer "F.Cu") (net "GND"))
 (segment (start 164.4 121.64) (end 163.4 120.64) (width 0.2) (layer "F.Cu") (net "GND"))
 (segment (start 163.4 120.64) (end 161.4 120.64) (width 0.2) (layer "F.Cu") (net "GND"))
 (segment (start 119.25 106.5) (end 118.61 105.86) (width 0.2) (layer "F.Cu") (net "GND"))
 (segment (start 118.61 105.86) (end 116.44 105.86) (width 0.2) (layer "F.Cu") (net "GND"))
 (segment (start 120.4 114.36) (end 126.75 120.71) (width 0.2) (layer "B.Cu") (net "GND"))
 (segment (start 116.44 105.86) (end 120.4 109.82) (width 0.2) (layer "B.Cu") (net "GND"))
 (segment (start 120.4 109.82) (end 120.4 114.36) (width 0.2) (layer "B.Cu") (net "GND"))
 (segment (start 157.23 101.77) (end 159.28 101.77) (width 0.2) (layer "B.Cu") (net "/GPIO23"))
 (segment (start 152.15 87.63) (end 154.9 90.38) (width 0.2) (layer "B.Cu") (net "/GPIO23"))
 (segment (start 154.9 99.44) (end 157.23 101.77) (width 0.2) (layer "B.Cu") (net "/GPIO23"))
 (segment (start 154.9 90.38) (end 154.9 99.44) (width 0.2) (layer "B.Cu") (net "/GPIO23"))
 (segment (start 161.5 98) (end 160.19 96.69) (width 0.2) (layer "F.Cu") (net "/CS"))
 (segment (start 160.19 96.69) (end 159.28 96.69) (width 0.2) (layer "F.Cu") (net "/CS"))
 (segment (start 152.15 105.41) (end 157.23 100.33) (width 0.2) (layer "F.Cu") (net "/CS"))
 (segment (start 157.23 100.33) (end 160.92 100.33) (width 0.2) (layer "F.Cu") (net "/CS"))
 (segment (start 160.92 100.33) (end 161.5 99.75) (width 0.2) (layer "F.Cu") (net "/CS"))
 (segment (start 161.5 99.75) (end 161.5 98) (width 0.2) (layer "F.Cu") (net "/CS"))
 (segment (start 155.79 99.23) (end 159.28 99.23) (width 0.2) (layer "F.Cu") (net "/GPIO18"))
 (segment (start 159.28 99.23) (end 159.33 99.28) (width 0.2) (layer "F.Cu") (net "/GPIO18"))
 (segment (start 152.15 102.87) (end 155.79 99.23) (width 0.2) (layer "F.Cu") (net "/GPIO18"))
 (segment (start 160.67 105.46) (end 166.9 99.23) (width 0.2) (layer "B.Cu") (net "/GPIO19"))
 (segment (start 157.28 105.46) (end 160.67 105.46) (width 0.2) (layer "B.Cu") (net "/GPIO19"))
 (segment (start 152.15 100.33) (end 157.28 105.46) (width 0.2) (layer "B.Cu") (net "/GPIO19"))
 (segment (start 116.44 98.24) (end 116.44 91.23) (width 0.2) (layer "F.Cu") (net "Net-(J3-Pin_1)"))
 (segment (start 116.44 91.23) (end 114.69 89.48) (width 0.2) (layer "F.Cu") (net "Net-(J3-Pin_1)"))
 (segment (start 109.15 92.48) (end 112.15 89.48) (width 0.2) (layer "F.Cu") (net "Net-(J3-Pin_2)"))
 (segment (start 111.36 99.51) (end 109.97 99.51) (width 0.2) (layer "F.Cu") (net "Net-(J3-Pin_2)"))
 (segment (start 109.15 98.69) (end 109.15 92.48) (width 0.2) (layer "F.Cu") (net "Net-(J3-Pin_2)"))
 (segment (start 109.97 99.51) (end 109.15 98.69) (width 0.2) (layer "F.Cu") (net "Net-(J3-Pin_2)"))
 (segment (start 113.94 103.28) (end 113.94 121.69) (width 0.2) (layer "F.Cu") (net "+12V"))
 (segment (start 116.44 100.78) (end 113.94 103.28) (width 0.2) (layer "F.Cu") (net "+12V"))
 (segment (start 165.15 89.99) (end 165.875 89.265) (width 0.2) (layer "F.Cu") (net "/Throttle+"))
 (segment (start 165.15 106.06) (end 165.15 89.99) (width 0.2) (layer "F.Cu") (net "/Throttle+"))
 (segment (start 159.28 111.93) (end 165.15 106.06) (width 0.2) (layer "F.Cu") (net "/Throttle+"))
 (segment (start 163.335 105.455) (end 163.335 89.265) (width 0.2) (layer "F.Cu") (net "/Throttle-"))
 (segment (start 159.28 109.39) (end 159.4 109.39) (width 0.2) (layer "F.Cu") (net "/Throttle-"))
 (segment (start 159.4 109.39) (end 163.335 105.455) (width 0.2) (layer "F.Cu") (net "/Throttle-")))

